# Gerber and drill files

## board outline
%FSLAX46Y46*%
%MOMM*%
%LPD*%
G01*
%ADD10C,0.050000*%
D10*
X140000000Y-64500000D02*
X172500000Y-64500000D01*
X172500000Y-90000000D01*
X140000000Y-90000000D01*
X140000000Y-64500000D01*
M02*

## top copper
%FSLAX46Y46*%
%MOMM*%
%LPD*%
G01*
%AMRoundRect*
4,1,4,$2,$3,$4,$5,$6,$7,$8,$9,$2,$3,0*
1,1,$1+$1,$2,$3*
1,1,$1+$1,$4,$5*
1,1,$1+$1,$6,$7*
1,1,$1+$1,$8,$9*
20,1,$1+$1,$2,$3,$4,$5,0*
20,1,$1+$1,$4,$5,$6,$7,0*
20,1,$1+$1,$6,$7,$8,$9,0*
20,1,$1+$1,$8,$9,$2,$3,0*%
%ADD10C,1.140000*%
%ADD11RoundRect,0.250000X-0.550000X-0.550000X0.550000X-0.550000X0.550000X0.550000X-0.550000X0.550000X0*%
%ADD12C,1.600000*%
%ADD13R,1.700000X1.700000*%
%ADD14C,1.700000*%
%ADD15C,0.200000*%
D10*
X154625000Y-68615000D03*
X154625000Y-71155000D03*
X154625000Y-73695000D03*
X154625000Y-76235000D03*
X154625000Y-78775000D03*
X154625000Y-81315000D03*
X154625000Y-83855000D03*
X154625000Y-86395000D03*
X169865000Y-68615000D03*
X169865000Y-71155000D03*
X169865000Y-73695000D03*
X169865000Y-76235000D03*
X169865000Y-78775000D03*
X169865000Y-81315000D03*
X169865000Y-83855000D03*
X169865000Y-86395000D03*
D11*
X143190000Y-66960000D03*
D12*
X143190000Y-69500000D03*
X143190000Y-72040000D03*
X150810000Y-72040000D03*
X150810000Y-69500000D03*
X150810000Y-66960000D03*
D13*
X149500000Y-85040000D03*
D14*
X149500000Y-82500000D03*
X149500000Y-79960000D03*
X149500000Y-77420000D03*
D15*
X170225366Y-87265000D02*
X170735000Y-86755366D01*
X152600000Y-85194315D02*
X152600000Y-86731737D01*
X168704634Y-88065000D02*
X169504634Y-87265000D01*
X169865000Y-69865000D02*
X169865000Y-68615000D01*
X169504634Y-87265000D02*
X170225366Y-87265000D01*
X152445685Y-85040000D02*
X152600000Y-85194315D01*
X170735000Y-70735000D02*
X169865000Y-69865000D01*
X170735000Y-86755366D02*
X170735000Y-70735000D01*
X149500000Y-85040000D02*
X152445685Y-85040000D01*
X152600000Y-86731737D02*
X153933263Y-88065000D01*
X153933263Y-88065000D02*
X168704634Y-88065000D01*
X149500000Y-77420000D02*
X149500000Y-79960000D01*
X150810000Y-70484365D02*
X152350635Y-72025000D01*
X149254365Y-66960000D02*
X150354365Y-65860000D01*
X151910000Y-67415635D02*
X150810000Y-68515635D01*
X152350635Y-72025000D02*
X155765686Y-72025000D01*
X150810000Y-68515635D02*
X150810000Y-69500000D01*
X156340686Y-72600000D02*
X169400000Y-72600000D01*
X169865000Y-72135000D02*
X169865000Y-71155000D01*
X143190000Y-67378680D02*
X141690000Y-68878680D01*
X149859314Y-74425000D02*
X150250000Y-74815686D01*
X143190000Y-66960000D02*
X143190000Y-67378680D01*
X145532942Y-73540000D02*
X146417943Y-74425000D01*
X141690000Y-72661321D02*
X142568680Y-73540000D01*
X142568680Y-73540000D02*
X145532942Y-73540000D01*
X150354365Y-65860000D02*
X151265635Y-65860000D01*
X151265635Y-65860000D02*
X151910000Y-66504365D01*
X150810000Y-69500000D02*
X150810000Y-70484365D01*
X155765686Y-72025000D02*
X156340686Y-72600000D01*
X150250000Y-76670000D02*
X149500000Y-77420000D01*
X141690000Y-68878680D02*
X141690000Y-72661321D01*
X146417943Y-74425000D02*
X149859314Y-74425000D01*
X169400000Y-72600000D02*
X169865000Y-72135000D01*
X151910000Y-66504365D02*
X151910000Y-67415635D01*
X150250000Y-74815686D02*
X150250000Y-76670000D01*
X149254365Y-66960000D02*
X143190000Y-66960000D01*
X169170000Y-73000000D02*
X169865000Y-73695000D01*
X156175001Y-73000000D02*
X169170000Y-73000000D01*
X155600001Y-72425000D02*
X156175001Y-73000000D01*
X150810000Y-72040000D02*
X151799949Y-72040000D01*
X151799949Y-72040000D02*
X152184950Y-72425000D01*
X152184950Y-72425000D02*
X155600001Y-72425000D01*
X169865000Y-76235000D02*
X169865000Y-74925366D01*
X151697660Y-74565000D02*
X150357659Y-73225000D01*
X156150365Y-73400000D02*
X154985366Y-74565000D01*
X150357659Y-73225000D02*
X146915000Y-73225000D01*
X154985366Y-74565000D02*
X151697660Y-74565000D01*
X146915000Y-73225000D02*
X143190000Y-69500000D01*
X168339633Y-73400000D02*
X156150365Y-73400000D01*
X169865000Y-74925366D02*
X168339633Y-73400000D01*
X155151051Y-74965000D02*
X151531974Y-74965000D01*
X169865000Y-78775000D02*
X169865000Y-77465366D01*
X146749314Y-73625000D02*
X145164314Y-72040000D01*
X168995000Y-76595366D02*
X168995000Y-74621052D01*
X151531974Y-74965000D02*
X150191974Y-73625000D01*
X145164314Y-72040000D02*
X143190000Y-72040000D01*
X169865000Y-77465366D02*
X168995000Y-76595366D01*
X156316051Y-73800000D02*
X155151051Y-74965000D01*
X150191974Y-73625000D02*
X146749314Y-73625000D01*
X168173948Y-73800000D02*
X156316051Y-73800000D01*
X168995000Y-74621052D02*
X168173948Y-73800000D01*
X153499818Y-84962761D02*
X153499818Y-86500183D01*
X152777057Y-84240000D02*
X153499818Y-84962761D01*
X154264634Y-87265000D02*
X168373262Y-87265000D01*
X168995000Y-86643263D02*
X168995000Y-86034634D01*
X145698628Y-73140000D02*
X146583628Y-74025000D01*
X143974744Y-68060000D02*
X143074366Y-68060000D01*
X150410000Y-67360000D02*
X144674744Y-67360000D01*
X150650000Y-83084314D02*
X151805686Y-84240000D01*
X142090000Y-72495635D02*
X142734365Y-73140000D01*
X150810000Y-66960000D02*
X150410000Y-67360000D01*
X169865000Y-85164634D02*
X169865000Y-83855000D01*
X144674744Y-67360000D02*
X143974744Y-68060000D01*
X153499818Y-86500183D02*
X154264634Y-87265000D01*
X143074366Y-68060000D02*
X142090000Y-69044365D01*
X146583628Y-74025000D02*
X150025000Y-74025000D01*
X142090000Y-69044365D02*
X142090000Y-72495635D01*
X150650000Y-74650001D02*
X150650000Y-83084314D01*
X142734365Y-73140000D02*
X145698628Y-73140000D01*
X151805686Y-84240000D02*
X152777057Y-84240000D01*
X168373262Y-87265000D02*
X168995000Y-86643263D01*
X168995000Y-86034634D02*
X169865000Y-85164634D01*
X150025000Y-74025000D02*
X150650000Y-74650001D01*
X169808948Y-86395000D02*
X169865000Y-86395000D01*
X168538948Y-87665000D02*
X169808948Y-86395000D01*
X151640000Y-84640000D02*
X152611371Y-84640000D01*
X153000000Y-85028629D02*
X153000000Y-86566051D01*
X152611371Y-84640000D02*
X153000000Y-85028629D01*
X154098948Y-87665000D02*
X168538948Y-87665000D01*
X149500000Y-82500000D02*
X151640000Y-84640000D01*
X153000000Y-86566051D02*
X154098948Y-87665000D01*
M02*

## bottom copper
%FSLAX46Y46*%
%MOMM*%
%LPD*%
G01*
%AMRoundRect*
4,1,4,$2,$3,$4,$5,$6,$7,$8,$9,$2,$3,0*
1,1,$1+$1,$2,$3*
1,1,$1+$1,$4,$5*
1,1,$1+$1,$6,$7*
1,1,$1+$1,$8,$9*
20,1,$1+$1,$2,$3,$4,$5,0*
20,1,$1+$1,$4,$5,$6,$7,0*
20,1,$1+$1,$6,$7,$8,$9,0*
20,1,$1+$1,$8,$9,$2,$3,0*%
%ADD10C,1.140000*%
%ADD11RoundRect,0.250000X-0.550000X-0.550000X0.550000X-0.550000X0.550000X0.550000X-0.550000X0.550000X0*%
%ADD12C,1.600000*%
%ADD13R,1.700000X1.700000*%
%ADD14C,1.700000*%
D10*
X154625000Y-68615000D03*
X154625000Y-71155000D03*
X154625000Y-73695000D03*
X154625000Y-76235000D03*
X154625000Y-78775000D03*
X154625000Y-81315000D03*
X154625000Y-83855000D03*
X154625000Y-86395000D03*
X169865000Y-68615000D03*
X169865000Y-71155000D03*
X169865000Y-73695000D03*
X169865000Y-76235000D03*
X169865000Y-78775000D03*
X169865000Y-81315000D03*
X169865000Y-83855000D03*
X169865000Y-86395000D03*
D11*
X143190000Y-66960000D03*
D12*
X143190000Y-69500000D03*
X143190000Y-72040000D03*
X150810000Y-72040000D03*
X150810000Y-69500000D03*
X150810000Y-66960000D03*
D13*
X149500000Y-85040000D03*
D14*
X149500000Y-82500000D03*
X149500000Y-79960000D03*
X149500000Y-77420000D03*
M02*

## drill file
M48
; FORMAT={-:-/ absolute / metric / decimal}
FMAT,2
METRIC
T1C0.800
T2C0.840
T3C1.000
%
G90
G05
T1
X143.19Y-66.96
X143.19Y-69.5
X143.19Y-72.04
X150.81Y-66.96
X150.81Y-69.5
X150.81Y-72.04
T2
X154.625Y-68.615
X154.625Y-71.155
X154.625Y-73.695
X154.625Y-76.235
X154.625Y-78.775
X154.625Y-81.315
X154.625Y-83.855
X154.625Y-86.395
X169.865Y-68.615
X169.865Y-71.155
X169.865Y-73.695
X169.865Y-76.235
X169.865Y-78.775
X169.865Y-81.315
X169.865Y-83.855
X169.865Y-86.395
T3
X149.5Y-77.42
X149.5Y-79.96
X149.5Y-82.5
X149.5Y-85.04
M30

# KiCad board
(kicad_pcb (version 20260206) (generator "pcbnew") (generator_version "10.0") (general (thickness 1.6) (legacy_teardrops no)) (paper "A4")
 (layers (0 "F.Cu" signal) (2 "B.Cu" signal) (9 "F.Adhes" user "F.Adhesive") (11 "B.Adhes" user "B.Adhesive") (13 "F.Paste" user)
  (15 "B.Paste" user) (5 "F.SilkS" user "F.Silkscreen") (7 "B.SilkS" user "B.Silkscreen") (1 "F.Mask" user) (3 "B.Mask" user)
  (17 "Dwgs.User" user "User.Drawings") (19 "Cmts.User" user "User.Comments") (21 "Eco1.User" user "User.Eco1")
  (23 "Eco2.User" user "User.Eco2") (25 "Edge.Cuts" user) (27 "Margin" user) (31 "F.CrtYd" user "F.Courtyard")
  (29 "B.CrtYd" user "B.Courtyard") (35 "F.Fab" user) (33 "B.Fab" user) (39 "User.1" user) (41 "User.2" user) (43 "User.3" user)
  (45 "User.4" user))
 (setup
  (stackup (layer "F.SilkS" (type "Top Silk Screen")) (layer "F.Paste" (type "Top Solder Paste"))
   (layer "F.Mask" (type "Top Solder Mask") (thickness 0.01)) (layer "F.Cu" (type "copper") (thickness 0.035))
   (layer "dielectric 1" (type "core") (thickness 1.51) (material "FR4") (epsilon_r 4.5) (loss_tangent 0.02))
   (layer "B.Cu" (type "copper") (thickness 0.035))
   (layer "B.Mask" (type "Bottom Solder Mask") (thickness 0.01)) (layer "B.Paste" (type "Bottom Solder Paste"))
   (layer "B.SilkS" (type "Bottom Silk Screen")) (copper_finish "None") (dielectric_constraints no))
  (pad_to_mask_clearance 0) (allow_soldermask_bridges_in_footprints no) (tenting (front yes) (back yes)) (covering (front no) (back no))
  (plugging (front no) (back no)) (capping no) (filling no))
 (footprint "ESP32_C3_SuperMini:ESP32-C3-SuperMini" (layer "F.Cu") (at 162.245 77.505)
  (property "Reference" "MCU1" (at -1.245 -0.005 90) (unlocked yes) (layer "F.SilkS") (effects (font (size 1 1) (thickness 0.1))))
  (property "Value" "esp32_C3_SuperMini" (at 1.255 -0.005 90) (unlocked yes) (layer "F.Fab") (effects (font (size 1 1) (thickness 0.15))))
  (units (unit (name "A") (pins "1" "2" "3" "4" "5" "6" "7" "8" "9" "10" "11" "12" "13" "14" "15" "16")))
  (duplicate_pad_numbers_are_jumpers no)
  (pad "1" thru_hole circle (at -7.62 -8.89) (size 1.14 1.14) (drill 0.84) (layers "*.Cu" "*.Mask") (remove_unused_layers no)
   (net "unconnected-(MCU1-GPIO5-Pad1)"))
  (pad "2" thru_hole circle (at -7.62 -6.35) (size 1.14 1.14) (drill 0.84) (layers "*.Cu" "*.Mask") (remove_unused_layers no)
   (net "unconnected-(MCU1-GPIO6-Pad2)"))
  (pad "3" thru_hole circle (at -7.62 -3.81) (size 1.14 1.14) (drill 0.84) (layers "*.Cu" "*.Mask") (remove_unused_layers no)
   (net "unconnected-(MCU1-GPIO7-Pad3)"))
  (pad "4" thru_hole circle (at -7.62 -1.27) (size 1.14 1.14) (drill 0.84) (layers "*.Cu" "*.Mask") (remove_unused_layers no)
   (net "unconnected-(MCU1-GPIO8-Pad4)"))
  (pad "5" thru_hole circle (at -7.62 1.27) (size 1.14 1.14) (drill 0.84) (layers "*.Cu" "*.Mask") (remove_unused_layers no)
   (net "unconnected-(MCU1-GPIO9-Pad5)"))
  (pad "6" thru_hole circle (at -7.62 3.81) (size 1.14 1.14) (drill 0.84) (layers "*.Cu" "*.Mask") (remove_unused_layers no)
   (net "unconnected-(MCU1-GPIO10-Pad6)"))
  (pad "7" thru_hole circle (at -7.62 6.35) (size 1.14 1.14) (drill 0.84) (layers "*.Cu" "*.Mask") (remove_unused_layers no)
   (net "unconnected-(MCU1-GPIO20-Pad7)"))
  (pad "8" thru_hole circle (at -7.62 8.89) (size 1.14 1.14) (drill 0.84) (layers "*.Cu" "*.Mask") (remove_unused_layers no)
   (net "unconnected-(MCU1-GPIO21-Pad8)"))
  (pad "9" thru_hole circle (at 7.62 -8.89) (size 1.14 1.14) (drill 0.84) (layers "*.Cu" "*.Mask") (remove_unused_layers no) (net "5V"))
  (pad "10" thru_hole circle (at 7.62 -6.35) (size 1.14 1.14) (drill 0.84) (layers "*.Cu" "*.Mask") (remove_unused_layers no) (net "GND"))
  (pad "11" thru_hole circle (at 7.62 -3.81) (size 1.14 1.14) (drill 0.84) (layers "*.Cu" "*.Mask") (remove_unused_layers no) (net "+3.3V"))
  (pad "12" thru_hole circle (at 7.62 -1.27) (size 1.14 1.14) (drill 0.84) (layers "*.Cu" "*.Mask") (remove_unused_layers no) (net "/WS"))
  (pad "13" thru_hole circle (at 7.62 1.27) (size 1.14 1.14) (drill 0.84) (layers "*.Cu" "*.Mask") (remove_unused_layers no) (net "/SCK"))
  (pad "14" thru_hole circle (at 7.62 3.81) (size 1.14 1.14) (drill 0.84) (layers "*.Cu" "*.Mask") (remove_unused_layers no)
   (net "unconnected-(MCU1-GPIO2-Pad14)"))
  (pad "15" thru_hole circle (at 7.62 6.35) (size 1.14 1.14) (drill 0.84) (layers "*.Cu" "*.Mask") (remove_unused_layers no) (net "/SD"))
  (pad "16" thru_hole circle (at 7.62 8.89) (size 1.14 1.14) (drill 0.84) (layers "*.Cu" "*.Mask") (remove_unused_layers no) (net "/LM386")))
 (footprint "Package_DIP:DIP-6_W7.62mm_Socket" (layer "F.Cu") (at 143.19 66.96)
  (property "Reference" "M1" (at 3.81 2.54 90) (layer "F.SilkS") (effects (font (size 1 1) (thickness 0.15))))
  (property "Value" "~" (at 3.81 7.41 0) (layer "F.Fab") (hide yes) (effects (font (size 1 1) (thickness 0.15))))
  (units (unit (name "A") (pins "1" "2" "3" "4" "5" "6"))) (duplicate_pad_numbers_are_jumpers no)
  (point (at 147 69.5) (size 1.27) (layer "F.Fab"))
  (pad "1" thru_hole roundrect (at 0 0) (size 1.6 1.6) (drill 0.8) (layers "*.Cu" "*.Mask") (remove_unused_layers no)
   (roundrect_rratio 0.15625) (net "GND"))
  (pad "2" thru_hole circle (at 0 2.54) (size 1.6 1.6) (drill 0.8) (layers "*.Cu" "*.Mask") (remove_unused_layers no) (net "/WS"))
  (pad "3" thru_hole circle (at 0 5.08) (size 1.6 1.6) (drill 0.8) (layers "*.Cu" "*.Mask") (remove_unused_layers no) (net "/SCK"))
  (pad "4" thru_hole circle (at 7.62 5.08) (size 1.6 1.6) (drill 0.8) (layers "*.Cu" "*.Mask") (remove_unused_layers no) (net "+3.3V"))
  (pad "5" thru_hole circle (at 7.62 2.54) (size 1.6 1.6) (drill 0.8) (layers "*.Cu" "*.Mask") (remove_unused_layers no) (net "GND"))
  (pad "6" thru_hole circle (at 7.62 0) (size 1.6 1.6) (drill 0.8) (layers "*.Cu" "*.Mask") (remove_unused_layers no) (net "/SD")))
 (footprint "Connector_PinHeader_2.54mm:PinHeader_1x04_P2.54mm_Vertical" (layer "F.Cu") (at 149.5 85.04 180)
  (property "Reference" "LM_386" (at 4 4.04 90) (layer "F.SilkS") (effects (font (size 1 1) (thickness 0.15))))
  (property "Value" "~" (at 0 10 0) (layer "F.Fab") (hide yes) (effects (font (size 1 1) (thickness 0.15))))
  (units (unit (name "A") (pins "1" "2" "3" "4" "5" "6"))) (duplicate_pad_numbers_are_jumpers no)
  (pad "1" thru_hole rect (at 0 0 180) (size 1.7 1.7) (drill 1) (layers "*.Cu" "*.Mask") (remove_unused_layers no) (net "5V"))
  (pad "2" thru_hole circle (at 0 2.54 180) (size 1.7 1.7) (drill 1) (layers "*.Cu" "*.Mask") (remove_unused_layers no) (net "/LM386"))
  (pad "3" thru_hole circle (at 0 5.08 180) (size 1.7 1.7) (drill 1) (layers "*.Cu" "*.Mask") (remove_unused_layers no) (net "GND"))
  (pad "4" thru_hole circle (at 0 7.62 180) (size 1.7 1.7) (drill 1) (layers "*.Cu" "*.Mask") (remove_unused_layers no) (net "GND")))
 (gr_rect (start 140 64.5) (end 172.5 90) (stroke (width 0.05) (type default)) (fill no) (layer "Edge.Cuts"))
 (segment (start 170.225366 87.265) (end 170.735 86.755366) (width 0.2) (layer "F.Cu") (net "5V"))
 (segment (start 152.6 85.194315) (end 152.6 86.731737) (width 0.2) (layer "F.Cu") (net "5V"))
 (segment (start 168.704634 88.065) (end 169.504634 87.265) (width 0.2) (layer "F.Cu") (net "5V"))
 (segment (start 169.865 69.865) (end 169.865 68.615) (width 0.2) (layer "F.Cu") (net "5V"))
 (segment (start 169.504634 87.265) (end 170.225366 87.265) (width 0.2) (layer "F.Cu") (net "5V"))
 (segment (start 152.445685 85.04) (end 152.6 85.194315) (width 0.2) (layer "F.Cu") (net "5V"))
 (segment (start 170.735 70.735) (end 169.865 69.865) (width 0.2) (layer "F.Cu") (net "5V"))
 (segment (start 170.735 86.755366) (end 170.735 70.735) (width 0.2) (layer "F.Cu") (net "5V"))
 (segment (start 149.5 85.04) (end 152.445685 85.04) (width 0.2) (layer "F.Cu") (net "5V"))
 (segment (start 152.6 86.731737) (end 153.933263 88.065) (width 0.2) (layer "F.Cu") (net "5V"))
 (segment (start 153.933263 88.065) (end 168.704634 88.065) (width 0.2) (layer "F.Cu") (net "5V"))
 (segment (start 149.5 77.42) (end 149.5 79.96) (width 0.2) (layer "F.Cu") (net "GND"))
 (segment (start 150.81 70.484365) (end 152.350635 72.025) (width 0.2) (layer "F.Cu") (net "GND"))
 (segment (start 149.254365 66.96) (end 150.354365 65.86) (width 0.2) (layer "F.Cu") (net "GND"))
 (segment (start 151.91 67.415635) (end 150.81 68.515635) (width 0.2) (layer "F.Cu") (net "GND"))
 (segment (start 152.350635 72.025) (end 155.765686 72.025) (width 0.2) (layer "F.Cu") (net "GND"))
 (segment (start 150.81 68.515635) (end 150.81 69.5) (width 0.2) (layer "F.Cu") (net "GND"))
 (segment (start 156.340686 72.6) (end 169.4 72.6) (width 0.2) (layer "F.Cu") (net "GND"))
 (segment (start 169.865 72.135) (end 169.865 71.155) (width 0.2) (layer "F.Cu") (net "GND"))
 (segment (start 143.19 67.37868) (end 141.69 68.87868) (width 0.2) (layer "F.Cu") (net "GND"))
 (segment (start 149.859314 74.425) (end 150.25 74.815686) (width 0.2) (layer "F.Cu") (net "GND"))
 (segment (start 143.19 66.96) (end 143.19 67.37868) (width 0.2) (layer "F.Cu") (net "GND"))
 (segment (start 145.532942 73.54) (end 146.417943 74.425) (width 0.2) (layer "F.Cu") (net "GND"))
 (segment (start 141.69 72.661321) (end 142.56868 73.54) (width 0.2) (layer "F.Cu") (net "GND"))
 (segment (start 142.56868 73.54) (end 145.532942 73.54) (width 0.2) (layer "F.Cu") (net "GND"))
 (segment (start 150.354365 65.86) (end 151.265635 65.86) (width 0.2) (layer "F.Cu") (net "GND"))
 (segment (start 151.265635 65.86) (end 151.91 66.504365) (width 0.2) (layer "F.Cu") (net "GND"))
 (segment (start 150.81 69.5) (end 150.81 70.484365) (width 0.2) (layer "F.Cu") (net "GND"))
 (segment (start 155.765686 72.025) (end 156.340686 72.6) (width 0.2) (layer "F.Cu") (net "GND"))
 (segment (start 150.25 76.67) (end 149.5 77.42) (width 0.2) (layer "F.Cu") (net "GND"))
 (segment (start 141.69 68.87868) (end 141.69 72.661321) (width 0.2) (layer "F.Cu") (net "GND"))
 (segment (start 146.417943 74.425) (end 149.859314 74.425) (width 0.2) (layer "F.Cu") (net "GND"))
 (segment (start 169.4 72.6) (end 169.865 72.135) (width 0.2) (layer "F.Cu") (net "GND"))
 (segment (start 151.91 66.504365) (end 151.91 67.415635) (width 0.2) (layer "F.Cu") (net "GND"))
 (segment (start 150.25 74.815686) (end 150.25 76.67) (width 0.2) (layer "F.Cu") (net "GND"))
 (segment (start 149.254365 66.96) (end 143.19 66.96) (width 0.2) (layer "F.Cu") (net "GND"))
 (segment (start 169.17 73) (end 169.865 73.695) (width 0.2) (layer "F.Cu") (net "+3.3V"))
 (segment (start 156.175001 73) (end 169.17 73) (width 0.2) (layer "F.Cu") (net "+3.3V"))
 (segment (start 155.600001 72.425) (end 156.175001 73) (width 0.2) (layer "F.Cu") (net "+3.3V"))
 (segment (start 150.81 72.04) (end 151.799949 72.04) (width 0.2) (layer "F.Cu") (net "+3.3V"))
 (segment (start 151.799949 72.04) (end 152.18495 72.425) (width 0.2) (layer "F.Cu") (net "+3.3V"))
 (segment (start 152.18495 72.425) (end 155.600001 72.425) (width 0.2) (layer "F.Cu") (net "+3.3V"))
 (segment (start 169.865 76.235) (end 169.865 74.925366) (width 0.2) (layer "F.Cu") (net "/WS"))
 (segment (start 151.69766 74.565) (end 150.357659 73.225) (width 0.2) (layer "F.Cu") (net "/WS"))
 (segment (start 156.150365 73.4) (end 154.985366 74.565) (width 0.2) (layer "F.Cu") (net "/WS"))
 (segment (start 150.357659 73.225) (end 146.915 73.225) (width 0.2) (layer "F.Cu") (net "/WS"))
 (segment (start 154.985366 74.565) (end 151.69766 74.565) (width 0.2) (layer "F.Cu") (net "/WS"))
 (segment (start 146.915 73.225) (end 143.19 69.5) (width 0.2) (layer "F.Cu") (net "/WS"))
 (segment (start 168.339633 73.4) (end 156.150365 73.4) (width 0.2) (layer "F.Cu") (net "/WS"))
 (segment (start 169.865 74.925366) (end 168.339633 73.4) (width 0.2) (layer "F.Cu") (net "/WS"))
 (segment (start 155.151051 74.965) (end 151.531974 74.965) (width 0.2) (layer "F.Cu") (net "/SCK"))
 (segment (start 169.865 78.775) (end 169.865 77.465366) (width 0.2) (layer "F.Cu") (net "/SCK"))
 (segment (start 146.749314 73.625) (end 145.164314 72.04) (width 0.2) (layer "F.Cu") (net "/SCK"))
 (segment (start 168.995 76.595366) (end 168.995 74.621052) (width 0.2) (layer "F.Cu") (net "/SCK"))
 (segment (start 151.531974 74.965) (end 150.191974 73.625) (width 0.2) (layer "F.Cu") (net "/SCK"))
 (segment (start 145.164314 72.04) (end 143.19 72.04) (width 0.2) (layer "F.Cu") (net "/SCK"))
 (segment (start 169.865 77.465366) (end 168.995 76.595366) (width 0.2) (layer "F.Cu") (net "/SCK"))
 (segment (start 156.316051 73.8) (end 155.151051 74.965) (width 0.2) (layer "F.Cu") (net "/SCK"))
 (segment (start 150.191974 73.625) (end 146.749314 73.625) (width 0.2) (layer "F.Cu") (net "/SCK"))
 (segment (start 168.173948 73.8) (end 156.316051 73.8) (width 0.2) (layer "F.Cu") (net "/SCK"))
 (segment (start 168.995 74.621052) (end 168.173948 73.8) (width 0.2) (layer "F.Cu") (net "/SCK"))
 (segment (start 153.499818 84.962761) (end 153.499818 86.500183) (width 0.2) (layer "F.Cu") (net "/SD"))
 (segment (start 152.777057 84.24) (end 153.499818 84.962761) (width 0.2) (layer "F.Cu") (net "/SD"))
 (segment (start 154.264634 87.265) (end 168.373262 87.265) (width 0.2) (layer "F.Cu") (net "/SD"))
 (segment (start 168.995 86.643263) (end 168.995 86.034634) (width 0.2) (layer "F.Cu") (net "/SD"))
 (segment (start 145.698628 73.14) (end 146.583628 74.025) (width 0.2) (layer "F.Cu") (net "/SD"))
 (segment (start 143.974744 68.06) (end 143.074366 68.06) (width 0.2) (layer "F.Cu") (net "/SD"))
 (segment (start 150.41 67.36) (end 144.674744 67.36) (width 0.2) (layer "F.Cu") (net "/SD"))
 (segment (start 150.65 83.084314) (end 151.805686 84.24) (width 0.2) (layer "F.Cu") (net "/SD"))
 (segment (start 142.09 72.495635) (end 142.734365 73.14) (width 0.2) (layer "F.Cu") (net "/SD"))
 (segment (start 150.81 66.96) (end 150.41 67.36) (width 0.2) (layer "F.Cu") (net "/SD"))
 (segment (start 169.865 85.164634) (end 169.865 83.855) (width 0.2) (layer "F.Cu") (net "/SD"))
 (segment (start 144.674744 67.36) (end 143.974744 68.06) (width 0.2) (layer "F.Cu") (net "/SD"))
 (segment (start 153.499818 86.500183) (end 154.264634 87.265) (width 0.2) (layer "F.Cu") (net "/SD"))
 (segment (start 143.074366 68.06) (end 142.09 69.044365) (width 0.2) (layer "F.Cu") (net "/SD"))
 (segment (start 146.583628 74.025) (end 150.025 74.025) (width 0.2) (layer "F.Cu") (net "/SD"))
 (segment (start 142.09 69.044365) (end 142.09 72.495635) (width 0.2) (layer "F.Cu") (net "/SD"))
 (segment (start 150.65 74.650001) (end 150.65 83.084314) (width 0.2) (layer "F.Cu") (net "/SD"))
 (segment (start 142.734365 73.14) (end 145.698628 73.14) (width 0.2) (layer "F.Cu") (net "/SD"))
 (segment (start 151.805686 84.24) (end 152.777057 84.24) (width 0.2) (layer "F.Cu") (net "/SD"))
 (segment (start 168.373262 87.265) (end 168.995 86.643263) (width 0.2) (layer "F.Cu") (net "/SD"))
 (segment (start 168.995 86.034634) (end 169.865 85.164634) (width 0.2) (layer "F.Cu") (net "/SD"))
 (segment (start 150.025 74.025) (end 150.65 74.650001) (width 0.2) (layer "F.Cu") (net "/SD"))
 (segment (start 169.808948 86.395) (end 169.865 86.395) (width 0.2) (layer "F.Cu") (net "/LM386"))
 (segment (start 168.538948 87.665) (end 169.808948 86.395) (width 0.2) (layer "F.Cu") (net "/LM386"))
 (segment (start 151.64 84.64) (end 152.611371 84.64) (width 0.2) (layer "F.Cu") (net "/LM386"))
 (segment (start 153 85.028629) (end 153 86.566051) (width 0.2) (layer "F.Cu") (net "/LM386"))
 (segment (start 152.611371 84.64) (end 153 85.028629) (width 0.2) (layer "F.Cu") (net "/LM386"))
 (segment (start 154.098948 87.665) (end 168.538948 87.665) (width 0.2) (layer "F.Cu") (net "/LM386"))
 (segment (start 149.5 82.5) (end 151.64 84.64) (width 0.2) (layer "F.Cu") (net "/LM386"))
 (segment (start 153 86.566051) (end 154.098948 87.665) (width 0.2) (layer "F.Cu") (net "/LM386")))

